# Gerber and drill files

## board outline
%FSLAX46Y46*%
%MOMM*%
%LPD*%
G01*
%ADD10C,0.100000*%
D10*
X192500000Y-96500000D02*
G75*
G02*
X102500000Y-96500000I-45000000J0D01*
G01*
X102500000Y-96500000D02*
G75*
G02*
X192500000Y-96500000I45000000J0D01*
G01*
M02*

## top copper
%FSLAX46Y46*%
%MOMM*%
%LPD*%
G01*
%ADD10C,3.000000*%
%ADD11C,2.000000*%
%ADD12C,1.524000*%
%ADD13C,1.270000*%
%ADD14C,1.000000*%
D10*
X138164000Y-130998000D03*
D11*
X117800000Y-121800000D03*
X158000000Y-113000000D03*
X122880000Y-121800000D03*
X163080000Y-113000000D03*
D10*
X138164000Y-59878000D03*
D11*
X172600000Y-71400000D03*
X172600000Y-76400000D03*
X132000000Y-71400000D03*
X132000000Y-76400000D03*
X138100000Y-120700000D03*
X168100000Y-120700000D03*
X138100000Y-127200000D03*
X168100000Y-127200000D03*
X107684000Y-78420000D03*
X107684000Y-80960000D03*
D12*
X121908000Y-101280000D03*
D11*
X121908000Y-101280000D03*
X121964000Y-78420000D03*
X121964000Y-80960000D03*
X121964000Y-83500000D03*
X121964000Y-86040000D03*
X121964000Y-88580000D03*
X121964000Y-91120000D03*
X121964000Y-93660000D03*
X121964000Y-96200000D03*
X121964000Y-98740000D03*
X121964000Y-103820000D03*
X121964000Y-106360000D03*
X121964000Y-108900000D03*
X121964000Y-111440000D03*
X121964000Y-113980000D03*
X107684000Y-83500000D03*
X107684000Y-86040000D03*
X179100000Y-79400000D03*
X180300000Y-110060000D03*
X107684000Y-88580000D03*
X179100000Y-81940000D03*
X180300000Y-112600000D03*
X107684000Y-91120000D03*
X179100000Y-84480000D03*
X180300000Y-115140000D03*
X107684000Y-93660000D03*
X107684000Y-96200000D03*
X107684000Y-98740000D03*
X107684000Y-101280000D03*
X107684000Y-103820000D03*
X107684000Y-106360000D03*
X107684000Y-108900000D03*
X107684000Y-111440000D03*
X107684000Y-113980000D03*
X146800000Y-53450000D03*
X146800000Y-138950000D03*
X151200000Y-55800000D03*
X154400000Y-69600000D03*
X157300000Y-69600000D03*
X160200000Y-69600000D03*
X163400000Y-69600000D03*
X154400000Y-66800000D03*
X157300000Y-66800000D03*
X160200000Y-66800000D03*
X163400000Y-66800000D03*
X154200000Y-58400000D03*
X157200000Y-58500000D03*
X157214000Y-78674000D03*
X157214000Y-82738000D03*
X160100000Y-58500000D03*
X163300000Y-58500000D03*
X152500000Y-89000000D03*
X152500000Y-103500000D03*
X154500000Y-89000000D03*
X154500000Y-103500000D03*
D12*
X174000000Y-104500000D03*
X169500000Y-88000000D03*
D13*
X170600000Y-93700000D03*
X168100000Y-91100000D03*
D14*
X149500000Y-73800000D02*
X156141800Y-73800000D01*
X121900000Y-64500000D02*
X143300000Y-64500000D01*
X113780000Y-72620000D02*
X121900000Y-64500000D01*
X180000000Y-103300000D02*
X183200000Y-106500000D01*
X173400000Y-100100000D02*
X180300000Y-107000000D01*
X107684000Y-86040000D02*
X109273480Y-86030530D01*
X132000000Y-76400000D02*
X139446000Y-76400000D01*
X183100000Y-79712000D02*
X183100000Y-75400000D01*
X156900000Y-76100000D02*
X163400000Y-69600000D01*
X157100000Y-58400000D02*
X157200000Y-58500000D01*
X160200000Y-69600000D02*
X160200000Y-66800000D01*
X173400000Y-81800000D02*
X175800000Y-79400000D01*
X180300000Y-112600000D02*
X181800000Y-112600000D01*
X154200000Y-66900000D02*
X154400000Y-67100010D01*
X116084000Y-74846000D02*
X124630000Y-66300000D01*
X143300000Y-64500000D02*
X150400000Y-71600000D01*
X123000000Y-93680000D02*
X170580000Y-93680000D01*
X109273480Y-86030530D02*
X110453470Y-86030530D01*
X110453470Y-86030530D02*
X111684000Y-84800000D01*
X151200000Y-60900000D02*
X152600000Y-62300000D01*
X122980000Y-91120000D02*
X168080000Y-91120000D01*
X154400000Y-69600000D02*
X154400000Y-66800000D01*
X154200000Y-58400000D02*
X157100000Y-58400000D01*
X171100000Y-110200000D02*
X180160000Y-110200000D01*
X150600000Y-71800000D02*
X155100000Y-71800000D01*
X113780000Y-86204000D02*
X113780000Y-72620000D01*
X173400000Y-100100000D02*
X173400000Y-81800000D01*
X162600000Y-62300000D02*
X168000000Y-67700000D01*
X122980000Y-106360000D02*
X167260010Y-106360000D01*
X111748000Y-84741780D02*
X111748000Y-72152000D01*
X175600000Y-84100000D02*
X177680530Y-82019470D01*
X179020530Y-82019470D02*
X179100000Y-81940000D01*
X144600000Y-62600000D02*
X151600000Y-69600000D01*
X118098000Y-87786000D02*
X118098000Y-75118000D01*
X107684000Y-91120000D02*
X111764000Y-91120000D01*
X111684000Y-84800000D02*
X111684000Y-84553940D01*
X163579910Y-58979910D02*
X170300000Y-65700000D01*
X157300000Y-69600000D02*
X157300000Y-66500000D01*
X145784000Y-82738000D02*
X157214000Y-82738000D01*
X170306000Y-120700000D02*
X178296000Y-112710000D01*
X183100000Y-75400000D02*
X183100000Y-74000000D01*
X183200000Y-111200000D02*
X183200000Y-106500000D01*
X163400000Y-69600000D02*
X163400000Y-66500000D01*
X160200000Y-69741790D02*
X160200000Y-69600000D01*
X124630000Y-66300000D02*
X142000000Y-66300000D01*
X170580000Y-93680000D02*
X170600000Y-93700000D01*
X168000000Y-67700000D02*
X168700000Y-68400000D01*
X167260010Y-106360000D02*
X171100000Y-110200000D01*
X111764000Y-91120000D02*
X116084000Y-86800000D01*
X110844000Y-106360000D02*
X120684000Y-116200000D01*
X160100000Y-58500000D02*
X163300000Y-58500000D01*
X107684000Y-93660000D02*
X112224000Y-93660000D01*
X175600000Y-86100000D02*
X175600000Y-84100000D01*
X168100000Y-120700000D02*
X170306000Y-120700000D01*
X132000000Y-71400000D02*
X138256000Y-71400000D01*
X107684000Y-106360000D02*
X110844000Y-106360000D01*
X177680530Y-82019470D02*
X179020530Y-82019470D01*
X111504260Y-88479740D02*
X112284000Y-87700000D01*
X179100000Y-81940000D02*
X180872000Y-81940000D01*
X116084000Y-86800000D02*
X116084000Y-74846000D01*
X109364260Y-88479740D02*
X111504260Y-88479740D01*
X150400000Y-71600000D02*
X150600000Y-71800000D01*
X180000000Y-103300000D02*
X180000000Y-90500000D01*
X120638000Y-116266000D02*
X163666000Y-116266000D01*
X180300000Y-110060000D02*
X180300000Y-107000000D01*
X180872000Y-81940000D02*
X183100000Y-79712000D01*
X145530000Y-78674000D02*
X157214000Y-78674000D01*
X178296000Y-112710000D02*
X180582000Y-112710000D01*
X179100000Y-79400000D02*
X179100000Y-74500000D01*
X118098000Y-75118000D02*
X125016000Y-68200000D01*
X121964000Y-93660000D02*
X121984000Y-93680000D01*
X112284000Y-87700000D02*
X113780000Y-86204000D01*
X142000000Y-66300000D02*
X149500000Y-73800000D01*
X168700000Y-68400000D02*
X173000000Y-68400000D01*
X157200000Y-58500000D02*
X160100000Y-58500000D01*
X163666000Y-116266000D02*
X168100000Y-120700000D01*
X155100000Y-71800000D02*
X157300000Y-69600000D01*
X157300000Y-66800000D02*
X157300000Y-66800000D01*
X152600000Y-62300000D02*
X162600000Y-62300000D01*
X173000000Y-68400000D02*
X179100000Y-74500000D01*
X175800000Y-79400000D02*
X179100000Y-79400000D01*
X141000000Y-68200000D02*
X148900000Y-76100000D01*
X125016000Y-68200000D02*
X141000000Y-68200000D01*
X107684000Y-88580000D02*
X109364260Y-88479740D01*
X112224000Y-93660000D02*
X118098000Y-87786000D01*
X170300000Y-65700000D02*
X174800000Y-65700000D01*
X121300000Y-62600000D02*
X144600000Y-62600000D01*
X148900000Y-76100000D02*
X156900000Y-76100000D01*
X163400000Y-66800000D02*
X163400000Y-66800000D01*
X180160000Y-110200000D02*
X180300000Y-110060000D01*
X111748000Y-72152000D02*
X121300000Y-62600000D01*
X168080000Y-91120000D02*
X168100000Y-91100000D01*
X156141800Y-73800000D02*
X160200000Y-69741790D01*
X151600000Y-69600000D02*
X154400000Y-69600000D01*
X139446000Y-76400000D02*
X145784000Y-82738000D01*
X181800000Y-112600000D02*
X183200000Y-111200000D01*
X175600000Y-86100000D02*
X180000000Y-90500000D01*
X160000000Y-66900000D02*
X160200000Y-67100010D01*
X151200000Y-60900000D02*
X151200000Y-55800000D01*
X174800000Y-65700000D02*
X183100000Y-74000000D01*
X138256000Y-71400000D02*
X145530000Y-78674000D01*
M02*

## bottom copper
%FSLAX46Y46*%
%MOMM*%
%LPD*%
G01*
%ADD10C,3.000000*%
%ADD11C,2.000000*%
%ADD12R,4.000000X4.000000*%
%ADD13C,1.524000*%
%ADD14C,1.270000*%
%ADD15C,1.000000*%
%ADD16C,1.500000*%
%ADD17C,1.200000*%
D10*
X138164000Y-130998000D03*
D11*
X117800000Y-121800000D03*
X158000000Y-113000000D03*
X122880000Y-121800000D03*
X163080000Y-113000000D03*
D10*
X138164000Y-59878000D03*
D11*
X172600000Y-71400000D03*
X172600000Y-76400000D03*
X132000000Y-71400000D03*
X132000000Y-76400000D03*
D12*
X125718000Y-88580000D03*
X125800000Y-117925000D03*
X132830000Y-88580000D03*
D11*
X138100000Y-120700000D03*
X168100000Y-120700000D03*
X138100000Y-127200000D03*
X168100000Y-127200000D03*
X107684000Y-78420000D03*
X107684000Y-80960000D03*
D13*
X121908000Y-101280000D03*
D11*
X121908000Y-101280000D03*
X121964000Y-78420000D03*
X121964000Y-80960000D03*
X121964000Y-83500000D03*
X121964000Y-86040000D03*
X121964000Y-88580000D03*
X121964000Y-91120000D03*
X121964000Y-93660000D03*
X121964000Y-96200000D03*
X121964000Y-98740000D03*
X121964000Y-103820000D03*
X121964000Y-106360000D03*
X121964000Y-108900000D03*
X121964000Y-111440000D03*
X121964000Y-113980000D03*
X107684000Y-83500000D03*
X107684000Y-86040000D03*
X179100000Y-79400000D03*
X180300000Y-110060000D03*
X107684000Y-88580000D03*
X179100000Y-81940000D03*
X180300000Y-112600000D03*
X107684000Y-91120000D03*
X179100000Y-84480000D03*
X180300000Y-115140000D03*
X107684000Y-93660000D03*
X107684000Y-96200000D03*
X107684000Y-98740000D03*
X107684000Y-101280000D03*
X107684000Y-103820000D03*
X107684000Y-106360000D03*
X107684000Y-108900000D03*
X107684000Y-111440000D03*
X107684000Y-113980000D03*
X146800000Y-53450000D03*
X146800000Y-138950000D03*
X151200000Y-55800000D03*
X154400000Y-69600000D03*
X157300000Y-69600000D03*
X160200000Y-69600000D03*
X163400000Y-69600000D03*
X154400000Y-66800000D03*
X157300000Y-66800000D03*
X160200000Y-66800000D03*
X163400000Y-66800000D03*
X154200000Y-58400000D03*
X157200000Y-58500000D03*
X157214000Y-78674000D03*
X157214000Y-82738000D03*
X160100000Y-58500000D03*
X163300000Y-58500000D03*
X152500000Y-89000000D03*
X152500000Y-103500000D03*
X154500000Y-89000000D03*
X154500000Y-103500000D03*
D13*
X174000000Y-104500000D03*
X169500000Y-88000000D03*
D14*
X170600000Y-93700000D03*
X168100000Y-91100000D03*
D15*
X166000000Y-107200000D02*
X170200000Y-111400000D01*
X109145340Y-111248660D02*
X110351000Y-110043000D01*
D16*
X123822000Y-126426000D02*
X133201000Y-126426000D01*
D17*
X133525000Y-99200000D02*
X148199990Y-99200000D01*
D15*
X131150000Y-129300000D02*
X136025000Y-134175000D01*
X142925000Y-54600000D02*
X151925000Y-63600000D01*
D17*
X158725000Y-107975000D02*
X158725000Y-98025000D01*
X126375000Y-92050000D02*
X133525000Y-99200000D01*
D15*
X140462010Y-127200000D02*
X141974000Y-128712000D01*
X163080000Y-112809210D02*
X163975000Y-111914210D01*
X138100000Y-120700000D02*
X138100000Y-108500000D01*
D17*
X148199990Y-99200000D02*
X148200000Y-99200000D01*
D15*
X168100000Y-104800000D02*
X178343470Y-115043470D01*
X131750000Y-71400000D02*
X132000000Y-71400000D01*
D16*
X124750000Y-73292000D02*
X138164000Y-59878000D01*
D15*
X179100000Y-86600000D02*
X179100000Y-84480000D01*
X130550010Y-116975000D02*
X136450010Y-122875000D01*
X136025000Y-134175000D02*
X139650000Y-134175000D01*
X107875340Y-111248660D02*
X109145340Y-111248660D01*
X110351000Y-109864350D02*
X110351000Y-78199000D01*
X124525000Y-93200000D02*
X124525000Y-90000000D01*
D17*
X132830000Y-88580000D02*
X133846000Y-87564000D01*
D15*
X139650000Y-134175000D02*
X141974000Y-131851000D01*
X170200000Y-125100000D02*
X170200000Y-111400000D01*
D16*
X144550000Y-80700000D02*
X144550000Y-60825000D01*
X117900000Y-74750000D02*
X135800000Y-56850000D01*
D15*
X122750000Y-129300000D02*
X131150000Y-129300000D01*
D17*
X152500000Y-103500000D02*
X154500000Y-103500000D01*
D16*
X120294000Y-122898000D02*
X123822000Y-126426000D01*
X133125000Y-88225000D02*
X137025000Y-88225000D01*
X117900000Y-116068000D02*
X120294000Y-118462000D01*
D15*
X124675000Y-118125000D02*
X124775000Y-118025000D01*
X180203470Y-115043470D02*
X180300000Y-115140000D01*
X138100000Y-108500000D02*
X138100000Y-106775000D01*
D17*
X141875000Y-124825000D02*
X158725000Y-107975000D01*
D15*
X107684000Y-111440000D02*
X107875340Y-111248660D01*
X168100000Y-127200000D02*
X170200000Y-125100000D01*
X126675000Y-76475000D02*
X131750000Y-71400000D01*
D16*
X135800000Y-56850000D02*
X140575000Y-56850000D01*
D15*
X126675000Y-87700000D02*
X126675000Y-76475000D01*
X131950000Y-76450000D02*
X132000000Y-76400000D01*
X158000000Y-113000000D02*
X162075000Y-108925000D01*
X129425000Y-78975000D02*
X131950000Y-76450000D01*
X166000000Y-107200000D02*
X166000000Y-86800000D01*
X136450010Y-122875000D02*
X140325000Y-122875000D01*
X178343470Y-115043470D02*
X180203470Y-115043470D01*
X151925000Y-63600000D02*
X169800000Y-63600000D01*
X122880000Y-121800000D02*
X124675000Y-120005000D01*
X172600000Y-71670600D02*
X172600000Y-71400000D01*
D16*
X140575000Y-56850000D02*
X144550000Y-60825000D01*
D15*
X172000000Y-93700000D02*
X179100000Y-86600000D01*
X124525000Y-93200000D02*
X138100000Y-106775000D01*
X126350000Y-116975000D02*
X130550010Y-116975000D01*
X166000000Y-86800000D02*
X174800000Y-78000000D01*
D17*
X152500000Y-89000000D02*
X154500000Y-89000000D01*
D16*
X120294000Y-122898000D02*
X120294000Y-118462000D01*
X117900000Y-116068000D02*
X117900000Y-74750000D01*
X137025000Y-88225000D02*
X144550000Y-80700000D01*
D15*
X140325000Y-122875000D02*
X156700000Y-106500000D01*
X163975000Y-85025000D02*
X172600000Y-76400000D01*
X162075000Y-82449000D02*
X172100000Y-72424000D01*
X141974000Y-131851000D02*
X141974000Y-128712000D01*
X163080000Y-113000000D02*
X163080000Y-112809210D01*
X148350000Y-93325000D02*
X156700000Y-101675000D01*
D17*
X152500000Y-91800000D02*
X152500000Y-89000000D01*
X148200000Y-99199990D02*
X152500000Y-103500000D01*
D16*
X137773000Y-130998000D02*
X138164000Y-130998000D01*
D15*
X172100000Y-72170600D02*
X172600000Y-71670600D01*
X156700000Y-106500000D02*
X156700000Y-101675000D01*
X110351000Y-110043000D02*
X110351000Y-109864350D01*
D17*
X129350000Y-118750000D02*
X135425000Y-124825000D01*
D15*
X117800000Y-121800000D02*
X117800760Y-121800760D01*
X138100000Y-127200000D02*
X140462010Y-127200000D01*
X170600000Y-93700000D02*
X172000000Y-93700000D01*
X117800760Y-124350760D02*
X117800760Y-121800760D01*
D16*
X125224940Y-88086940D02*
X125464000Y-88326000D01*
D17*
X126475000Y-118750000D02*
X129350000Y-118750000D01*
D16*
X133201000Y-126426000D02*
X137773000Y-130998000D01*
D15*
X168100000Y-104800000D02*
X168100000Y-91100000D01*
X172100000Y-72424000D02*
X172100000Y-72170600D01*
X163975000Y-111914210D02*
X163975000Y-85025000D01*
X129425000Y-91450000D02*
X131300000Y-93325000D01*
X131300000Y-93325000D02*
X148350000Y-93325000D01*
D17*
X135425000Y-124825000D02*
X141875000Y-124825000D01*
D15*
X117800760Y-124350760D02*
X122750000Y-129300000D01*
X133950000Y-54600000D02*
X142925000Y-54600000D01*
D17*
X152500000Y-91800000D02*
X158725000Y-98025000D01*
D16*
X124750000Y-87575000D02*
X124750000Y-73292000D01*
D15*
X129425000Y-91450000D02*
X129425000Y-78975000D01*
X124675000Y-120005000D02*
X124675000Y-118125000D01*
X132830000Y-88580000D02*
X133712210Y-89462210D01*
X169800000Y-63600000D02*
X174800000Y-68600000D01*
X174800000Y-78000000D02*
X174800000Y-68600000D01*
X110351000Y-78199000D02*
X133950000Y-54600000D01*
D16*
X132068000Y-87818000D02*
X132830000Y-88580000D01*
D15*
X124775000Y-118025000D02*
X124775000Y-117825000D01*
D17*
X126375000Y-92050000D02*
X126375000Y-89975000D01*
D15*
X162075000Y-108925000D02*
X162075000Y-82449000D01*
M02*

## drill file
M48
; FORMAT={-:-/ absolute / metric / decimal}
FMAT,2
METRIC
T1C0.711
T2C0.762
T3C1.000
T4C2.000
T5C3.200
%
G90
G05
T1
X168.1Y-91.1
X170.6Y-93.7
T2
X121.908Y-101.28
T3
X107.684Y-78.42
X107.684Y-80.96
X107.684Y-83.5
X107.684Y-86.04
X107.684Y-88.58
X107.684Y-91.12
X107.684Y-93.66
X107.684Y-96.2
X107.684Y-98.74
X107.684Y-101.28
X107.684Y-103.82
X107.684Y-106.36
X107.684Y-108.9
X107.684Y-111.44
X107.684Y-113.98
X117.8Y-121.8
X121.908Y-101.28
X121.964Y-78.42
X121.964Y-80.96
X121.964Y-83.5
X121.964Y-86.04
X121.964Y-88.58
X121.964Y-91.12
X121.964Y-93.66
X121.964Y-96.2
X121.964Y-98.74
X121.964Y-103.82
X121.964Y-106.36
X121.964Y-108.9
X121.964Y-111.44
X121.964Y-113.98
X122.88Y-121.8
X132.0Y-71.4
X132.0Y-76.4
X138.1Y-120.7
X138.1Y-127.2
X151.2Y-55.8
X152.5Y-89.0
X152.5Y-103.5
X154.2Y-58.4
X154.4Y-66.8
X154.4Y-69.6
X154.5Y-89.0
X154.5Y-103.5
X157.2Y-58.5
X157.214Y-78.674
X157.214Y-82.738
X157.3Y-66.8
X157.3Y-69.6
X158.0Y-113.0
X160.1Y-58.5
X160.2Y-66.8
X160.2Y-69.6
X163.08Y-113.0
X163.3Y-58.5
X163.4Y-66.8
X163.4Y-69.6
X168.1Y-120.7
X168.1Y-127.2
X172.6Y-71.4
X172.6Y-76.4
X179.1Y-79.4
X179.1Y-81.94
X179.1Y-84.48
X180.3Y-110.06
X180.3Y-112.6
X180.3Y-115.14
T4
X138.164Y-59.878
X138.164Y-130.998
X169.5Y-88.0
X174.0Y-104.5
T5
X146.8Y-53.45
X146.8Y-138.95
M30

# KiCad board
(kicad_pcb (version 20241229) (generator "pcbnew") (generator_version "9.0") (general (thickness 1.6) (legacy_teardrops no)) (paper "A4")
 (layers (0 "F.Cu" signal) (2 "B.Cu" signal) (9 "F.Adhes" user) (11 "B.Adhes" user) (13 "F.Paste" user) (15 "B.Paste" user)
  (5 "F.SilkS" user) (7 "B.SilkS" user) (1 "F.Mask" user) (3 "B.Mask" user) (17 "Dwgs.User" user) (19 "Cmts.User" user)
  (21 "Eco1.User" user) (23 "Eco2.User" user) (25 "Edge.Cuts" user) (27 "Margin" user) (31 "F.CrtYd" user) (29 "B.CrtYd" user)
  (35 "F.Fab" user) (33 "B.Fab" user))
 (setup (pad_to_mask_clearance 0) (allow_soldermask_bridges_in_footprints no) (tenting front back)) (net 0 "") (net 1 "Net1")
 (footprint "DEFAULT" (layer "F.Cu") (at 51.8 171.2)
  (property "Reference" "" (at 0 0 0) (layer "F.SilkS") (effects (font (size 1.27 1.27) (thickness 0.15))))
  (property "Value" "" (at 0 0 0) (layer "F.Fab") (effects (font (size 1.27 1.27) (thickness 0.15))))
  (pad "" thru_hole circle (at 86.364 -40.202) (size 3 3) (drill 2) (layers "*.Cu") (remove_unused_layers no))
  (pad "105" thru_hole circle (at 66 -49.4) (size 2 2) (drill 1) (layers "*.Cu") (remove_unused_layers no))
  (pad "105" thru_hole circle (at 106.2 -58.2) (size 2 2) (drill 1) (layers "*.Cu") (remove_unused_layers no))
  (pad "107" thru_hole circle (at 71.08 -49.4) (size 2 2) (drill 1) (layers "*.Cu") (remove_unused_layers no))
  (pad "107" thru_hole circle (at 111.28 -58.2) (size 2 2) (drill 1) (layers "*.Cu") (remove_unused_layers no))
  (pad "128" thru_hole circle (at 86.364 -111.322) (size 3 3) (drill 2) (layers "*.Cu") (remove_unused_layers no))
  (pad "129" thru_hole circle (at 120.8 -99.8 270) (size 2 2) (drill 1) (layers "*.Cu") (remove_unused_layers no))
  (pad "130" thru_hole circle (at 120.8 -94.8 270) (size 2 2) (drill 1) (layers "*.Cu") (remove_unused_layers no))
  (pad "131" thru_hole circle (at 80.2 -99.8 270) (size 2 2) (drill 1) (layers "*.Cu") (remove_unused_layers no))
  (pad "132" thru_hole circle (at 80.2 -94.8 270) (size 2 2) (drill 1) (layers "*.Cu") (remove_unused_layers no))
  (pad "134" smd rect (at 73.918 -82.62) (size 4 4) (layers "B.Cu"))
  (pad "134" smd rect (at 74 -53.275) (size 4 4) (layers "B.Cu"))
  (pad "134" smd rect (at 81.03 -82.62) (size 4 4) (layers "B.Cu"))
  (pad "137" thru_hole circle (at 86.3 -50.5 270) (size 2 2) (drill 1) (layers "*.Cu") (remove_unused_layers no))
  (pad "137" thru_hole circle (at 116.3 -50.5 270) (size 2 2) (drill 1) (layers "*.Cu") (remove_unused_layers no))
  (pad "138" thru_hole circle (at 86.3 -44 270) (size 2 2) (drill 1) (layers "*.Cu") (remove_unused_layers no))
  (pad "138" thru_hole circle (at 116.3 -44 270) (size 2 2) (drill 1) (layers "*.Cu") (remove_unused_layers no))
  (pad "141" thru_hole circle (at 55.884 -92.78) (size 2 2) (drill 1) (layers "*.Cu") (remove_unused_layers no))
  (pad "141" thru_hole circle (at 55.884 -90.24) (size 2 2) (drill 1) (layers "*.Cu") (remove_unused_layers no))
  (pad "141" thru_hole circle (at 70.108 -69.92) (size 1.524 1.524) (drill 0.762) (layers "*.Cu") (remove_unused_layers no))
  (pad "141" thru_hole circle (at 70.108 -69.92) (size 2 2) (drill 1) (layers "*.Cu") (remove_unused_layers no))
  (pad "141" thru_hole circle (at 70.164 -92.78) (size 2 2) (drill 1) (layers "*.Cu") (remove_unused_layers no))
  (pad "141" thru_hole circle (at 70.164 -90.24) (size 2 2) (drill 1) (layers "*.Cu") (remove_unused_layers no))
  (pad "141" thru_hole circle (at 70.164 -87.7) (size 2 2) (drill 1) (layers "*.Cu") (remove_unused_layers no))
  (pad "141" thru_hole circle (at 70.164 -85.16) (size 2 2) (drill 1) (layers "*.Cu") (remove_unused_layers no))
  (pad "141" thru_hole circle (at 70.164 -82.62) (size 2 2) (drill 1) (layers "*.Cu") (remove_unused_layers no))
  (pad "141" thru_hole circle (at 70.164 -80.08) (size 2 2) (drill 1) (layers "*.Cu") (remove_unused_layers no))
  (pad "141" thru_hole circle (at 70.164 -77.54) (size 2 2) (drill 1) (layers "*.Cu") (remove_unused_layers no))
  (pad "141" thru_hole circle (at 70.164 -75) (size 2 2) (drill 1) (layers "*.Cu") (remove_unused_layers no))
  (pad "141" thru_hole circle (at 70.164 -72.46) (size 2 2) (drill 1) (layers "*.Cu") (remove_unused_layers no))
  (pad "141" thru_hole circle (at 70.164 -67.38) (size 2 2) (drill 1) (layers "*.Cu") (remove_unused_layers no))
  (pad "141" thru_hole circle (at 70.164 -64.84) (size 2 2) (drill 1) (layers "*.Cu") (remove_unused_layers no))
  (pad "141" thru_hole circle (at 70.164 -62.3) (size 2 2) (drill 1) (layers "*.Cu") (remove_unused_layers no))
  (pad "141" thru_hole circle (at 70.164 -59.76) (size 2 2) (drill 1) (layers "*.Cu") (remove_unused_layers no))
  (pad "141" thru_hole circle (at 70.164 -57.22) (size 2 2) (drill 1) (layers "*.Cu") (remove_unused_layers no))
  (pad "142" thru_hole circle (at 55.884 -87.7) (size 2 2) (drill 1) (layers "*.Cu") (remove_unused_layers no))
  (pad "143" thru_hole circle (at 55.884 -85.16) (size 2 2) (drill 1) (layers "*.Cu") (remove_unused_layers no))
  (pad "143" thru_hole circle (at 127.3 -91.8) (size 2 2) (drill 1) (layers "*.Cu") (remove_unused_layers no))
  (pad "143" thru_hole circle (at 128.5 -61.14) (size 2 2) (drill 1) (layers "*.Cu") (remove_unused_layers no))
  (pad "144" thru_hole circle (at 55.884 -82.62) (size 2 2) (drill 1) (layers "*.Cu") (remove_unused_layers no))
  (pad "144" thru_hole circle (at 127.3 -89.26) (size 2 2) (drill 1) (layers "*.Cu") (remove_unused_layers no))
  (pad "144" thru_hole circle (at 128.5 -58.6) (size 2 2) (drill 1) (layers "*.Cu") (remove_unused_layers no))
  (pad "145" thru_hole circle (at 55.884 -80.08) (size 2 2) (drill 1) (layers "*.Cu") (remove_unused_layers no))
  (pad "145" thru_hole circle (at 127.3 -86.72) (size 2 2) (drill 1) (layers "*.Cu") (remove_unused_layers no))
  (pad "145" thru_hole circle (at 128.5 -56.06) (size 2 2) (drill 1) (layers "*.Cu") (remove_unused_layers no))
  (pad "146" thru_hole circle (at 55.884 -77.54) (size 2 2) (drill 1) (layers "*.Cu") (remove_unused_layers no))
  (pad "147" thru_hole circle (at 55.884 -75) (size 2 2) (drill 1) (layers "*.Cu") (remove_unused_layers no))
  (pad "148" thru_hole circle (at 55.884 -72.46) (size 2 2) (drill 1) (layers "*.Cu") (remove_unused_layers no))
  (pad "149" thru_hole circle (at 55.884 -69.92) (size 2 2) (drill 1) (layers "*.Cu") (remove_unused_layers no))
  (pad "150" thru_hole circle (at 55.884 -67.38) (size 2 2) (drill 1) (layers "*.Cu") (remove_unused_layers no))
  (pad "151" thru_hole circle (at 55.884 -64.84) (size 2 2) (drill 1) (layers "*.Cu") (remove_unused_layers no))
  (pad "152" thru_hole circle (at 55.884 -62.3) (size 2 2) (drill 1) (layers "*.Cu") (remove_unused_layers no))
  (pad "153" thru_hole circle (at 55.884 -59.76) (size 2 2) (drill 1) (layers "*.Cu") (remove_unused_layers no))
  (pad "154" thru_hole circle (at 55.884 -57.22) (size 2 2) (drill 1) (layers "*.Cu") (remove_unused_layers no))
  (pad "155" thru_hole circle (at 95 -117.75) (size 2 2) (drill 3.2) (layers "*.Cu") (remove_unused_layers no))
  (pad "155" thru_hole circle (at 95 -32.25) (size 2 2) (drill 3.2) (layers "*.Cu") (remove_unused_layers no))
  (pad "155" thru_hole circle (at 99.4 -115.4) (size 2 2) (drill 1) (layers "*.Cu") (remove_unused_layers no))
  (pad "156" thru_hole circle (at 102.6 -101.6) (size 2 2) (drill 1) (layers "*.Cu") (remove_unused_layers no))
  (pad "156" thru_hole circle (at 105.5 -101.6) (size 2 2) (drill 1) (layers "*.Cu") (remove_unused_layers no))
  (pad "156" thru_hole circle (at 108.4 -101.6) (size 2 2) (drill 1) (layers "*.Cu") (remove_unused_layers no))
  (pad "156" thru_hole circle (at 111.6 -101.6) (size 2 2) (drill 1) (layers "*.Cu") (remove_unused_layers no))
  (pad "157" thru_hole circle (at 102.6 -104.4) (size 2 2) (drill 1) (layers "*.Cu") (remove_unused_layers no))
  (pad "157" thru_hole circle (at 105.5 -104.4) (size 2 2) (drill 1) (layers "*.Cu") (remove_unused_layers no))
  (pad "157" thru_hole circle (at 108.4 -104.4) (size 2 2) (drill 1) (layers "*.Cu") (remove_unused_layers no))
  (pad "157" thru_hole circle (at 111.6 -104.4) (size 2 2) (drill 1) (layers "*.Cu") (remove_unused_layers no))
  (pad "158" thru_hole circle (at 102.4 -112.8) (size 2 2) (drill 1) (layers "*.Cu") (remove_unused_layers no))
  (pad "158" thru_hole circle (at 105.4 -112.7) (size 2 2) (drill 1) (layers "*.Cu") (remove_unused_layers no))
  (pad "158" thru_hole circle (at 105.414 -92.526) (size 2 2) (drill 1) (layers "*.Cu") (remove_unused_layers no))
  (pad "158" thru_hole circle (at 105.414 -88.462) (size 2 2) (drill 1) (layers "*.Cu") (remove_unused_layers no))
  (pad "158" thru_hole circle (at 108.3 -112.7) (size 2 2) (drill 1) (layers "*.Cu") (remove_unused_layers no))
  (pad "158" thru_hole circle (at 111.5 -112.7) (size 2 2) (drill 1) (layers "*.Cu") (remove_unused_layers no))
  (pad "169" thru_hole circle (at 100.7 -82.2) (size 2 2) (drill 1) (layers "*.Cu") (remove_unused_layers no))
  (pad "169" thru_hole circle (at 100.7 -67.7) (size 2 2) (drill 1) (layers "*.Cu") (remove_unused_layers no))
  (pad "170" thru_hole circle (at 102.7 -82.2) (size 2 2) (drill 1) (layers "*.Cu") (remove_unused_layers no))
  (pad "170" thru_hole circle (at 102.7 -67.7) (size 2 2) (drill 1) (layers "*.Cu") (remove_unused_layers no))
  (pad "171" thru_hole circle (at 122.2 -66.7) (size 1.524 1.524) (drill 2) (layers "*.Cu") (remove_unused_layers no))
  (pad "172" thru_hole circle (at 117.7 -83.2) (size 1.524 1.524) (drill 2) (layers "*.Cu") (remove_unused_layers no)))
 (gr_circle (center 147.5 96.5) (end 192.5 96.5) (stroke (width 0.1) (type solid)) (fill no) (layer "Edge.Cuts"))
 (segment (start 149.5 73.8) (end 156.1418 73.8) (width 1) (layer "F.Cu") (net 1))
 (segment (start 121.9 64.5) (end 143.3 64.5) (width 1) (layer "F.Cu") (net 1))
 (segment (start 113.78 72.62) (end 121.9 64.5) (width 1) (layer "F.Cu") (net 1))
 (segment (start 180 103.3) (end 183.2 106.5) (width 1) (layer "F.Cu") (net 1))
 (segment (start 173.4 100.1) (end 180.3 107) (width 1) (layer "F.Cu") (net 1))
 (segment (start 107.684 86.04) (end 109.27348 86.03053) (width 1) (layer "F.Cu") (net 1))
 (segment (start 132 76.4) (end 139.446 76.4) (width 1) (layer "F.Cu") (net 1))
 (segment (start 183.1 79.712) (end 183.1 75.4) (width 1) (layer "F.Cu") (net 1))
 (segment (start 156.9 76.1) (end 163.4 69.6) (width 1) (layer "F.Cu") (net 1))
 (segment (start 157.1 58.4) (end 157.2 58.5) (width 1) (layer "F.Cu") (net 1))
 (segment (start 160.2 69.6) (end 160.2 66.8) (width 1) (layer "F.Cu") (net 1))
 (segment (start 173.4 81.8) (end 175.8 79.4) (width 1) (layer "F.Cu") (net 1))
 (segment (start 180.3 112.6) (end 181.8 112.6) (width 1) (layer "F.Cu") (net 1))
 (segment (start 154.2 66.9) (end 154.4 67.10001) (width 1) (layer "F.Cu") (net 1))
 (segment (start 116.084 74.846) (end 124.63 66.3) (width 1) (layer "F.Cu") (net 1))
 (segment (start 143.3 64.5) (end 150.4 71.6) (width 1) (layer "F.Cu") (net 1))
 (segment (start 123 93.68) (end 170.58 93.68) (width 1) (layer "F.Cu") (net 1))
 (segment (start 109.27348 86.03053) (end 110.45347 86.03053) (width 1) (layer "F.Cu") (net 1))
 (segment (start 110.45347 86.03053) (end 111.684 84.8) (width 1) (layer "F.Cu") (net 1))
 (segment (start 151.2 60.9) (end 152.6 62.3) (width 1) (layer "F.Cu") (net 1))
 (segment (start 122.98 91.12) (end 168.08 91.12) (width 1) (layer "F.Cu") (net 1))
 (segment (start 154.4 69.6) (end 154.4 66.8) (width 1) (layer "F.Cu") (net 1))
 (segment (start 154.2 58.4) (end 157.1 58.4) (width 1) (layer "F.Cu") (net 1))
 (segment (start 171.1 110.2) (end 180.16 110.2) (width 1) (layer "F.Cu") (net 1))
 (segment (start 150.6 71.8) (end 155.1 71.8) (width 1) (layer "F.Cu") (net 1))
 (segment (start 113.78 86.204) (end 113.78 72.62) (width 1) (layer "F.Cu") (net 1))
 (segment (start 173.4 100.1) (end 173.4 81.8) (width 1) (layer "F.Cu") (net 1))
 (segment (start 162.6 62.3) (end 168 67.7) (width 1) (layer "F.Cu") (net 1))
 (segment (start 122.98 106.36) (end 167.26001 106.36) (width 1) (layer "F.Cu") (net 1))
 (segment (start 111.748 84.74178) (end 111.748 72.152) (width 1) (layer "F.Cu") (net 1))
 (segment (start 175.6 84.1) (end 177.68053 82.01947) (width 1) (layer "F.Cu") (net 1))
 (segment (start 179.02053 82.01947) (end 179.1 81.94) (width 1) (layer "F.Cu") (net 1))
 (segment (start 144.6 62.6) (end 151.6 69.6) (width 1) (layer "F.Cu") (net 1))
 (segment (start 118.098 87.786) (end 118.098 75.118) (width 1) (layer "F.Cu") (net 1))
 (segment (start 107.684 91.12) (end 111.764 91.12) (width 1) (layer "F.Cu") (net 1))
 (segment (start 111.684 84.8) (end 111.684 84.55394) (width 1) (layer "F.Cu") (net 1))
 (segment (start 163.57991 58.97991) (end 170.3 65.7) (width 1) (layer "F.Cu") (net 1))
 (segment (start 157.3 69.6) (end 157.3 66.5) (width 1) (layer "F.Cu") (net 1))
 (segment (start 145.784 82.738) (end 157.214 82.738) (width 1) (layer "F.Cu") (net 1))
 (segment (start 170.306 120.7) (end 178.296 112.71) (width 1) (layer "F.Cu") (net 1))
 (segment (start 183.1 75.4) (end 183.1 74) (width 1) (layer "F.Cu") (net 1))
 (segment (start 183.2 111.2) (end 183.2 106.5) (width 1) (layer "F.Cu") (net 1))
 (segment (start 163.4 69.6) (end 163.4 66.5) (width 1) (layer "F.Cu") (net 1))
 (segment (start 160.2 69.74179) (end 160.2 69.6) (width 1) (layer "F.Cu") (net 1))
 (segment (start 124.63 66.3) (end 142 66.3) (width 1) (layer "F.Cu") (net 1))
 (segment (start 170.58 93.68) (end 170.6 93.7) (width 1) (layer "F.Cu") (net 1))
 (segment (start 168 67.7) (end 168.7 68.4) (width 1) (layer "F.Cu") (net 1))
 (segment (start 167.26001 106.36) (end 171.1 110.2) (width 1) (layer "F.Cu") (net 1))
 (segment (start 111.764 91.12) (end 116.084 86.8) (width 1) (layer "F.Cu") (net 1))
 (segment (start 110.844 106.36) (end 120.684 116.2) (width 1) (layer "F.Cu") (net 1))
 (segment (start 160.1 58.5) (end 163.3 58.5) (width 1) (layer "F.Cu") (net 1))
 (segment (start 107.684 93.66) (end 112.224 93.66) (width 1) (layer "F.Cu") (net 1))
 (segment (start 175.6 86.1) (end 175.6 84.1) (width 1) (layer "F.Cu") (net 1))
 (segment (start 168.1 120.7) (end 170.306 120.7) (width 1) (layer "F.Cu") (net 1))
 (segment (start 132 71.4) (end 138.256 71.4) (width 1) (layer "F.Cu") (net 1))
 (segment (start 107.684 106.36) (end 110.844 106.36) (width 1) (layer "F.Cu") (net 1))
 (segment (start 177.68053 82.01947) (end 179.02053 82.01947) (width 1) (layer "F.Cu") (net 1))
 (segment (start 111.50426 88.47974) (end 112.284 87.7) (width 1) (layer "F.Cu") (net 1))
 (segment (start 179.1 81.94) (end 180.872 81.94) (width 1) (layer "F.Cu") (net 1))
 (segment (start 116.084 86.8) (end 116.084 74.846) (width 1) (layer "F.Cu") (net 1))
 (segment (start 109.36426 88.47974) (end 111.50426 88.47974) (width 1) (layer "F.Cu") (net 1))
 (segment (start 150.4 71.6) (end 150.6 71.8) (width 1) (layer "F.Cu") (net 1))
 (segment (start 180 103.3) (end 180 90.5) (width 1) (layer "F.Cu") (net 1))
 (segment (start 120.638 116.266) (end 163.666 116.266) (width 1) (layer "F.Cu") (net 1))
 (segment (start 180.3 110.06) (end 180.3 107) (width 1) (layer "F.Cu") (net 1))
 (segment (start 180.872 81.94) (end 183.1 79.712) (width 1) (layer "F.Cu") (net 1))
 (segment (start 145.53 78.674) (end 157.214 78.674) (width 1) (layer "F.Cu") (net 1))
 (segment (start 178.296 112.71) (end 180.582 112.71) (width 1) (layer "F.Cu") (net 1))
 (segment (start 179.1 79.4) (end 179.1 74.5) (width 1) (layer "F.Cu") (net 1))
 (segment (start 118.098 75.118) (end 125.016 68.2) (width 1) (layer "F.Cu") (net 1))
 (segment (start 121.964 93.66) (end 121.984 93.68) (width 1) (layer "F.Cu") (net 1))
 (segment (start 112.284 87.7) (end 113.78 86.204) (width 1) (layer "F.Cu") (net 1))
 (segment (start 142 66.3) (end 149.5 73.8) (width 1) (layer "F.Cu") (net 1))
 (segment (start 168.7 68.4) (end 173 68.4) (width 1) (layer "F.Cu") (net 1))
 (segment (start 157.2 58.5) (end 160.1 58.5) (width 1) (layer "F.Cu") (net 1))
 (segment (start 163.666 116.266) (end 168.1 120.7) (width 1) (layer "F.Cu") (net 1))
 (segment (start 155.1 71.8) (end 157.3 69.6) (width 1) (layer "F.Cu") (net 1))
 (segment (start 157.3 66.8) (end 157.3 66.8) (width 1) (layer "F.Cu") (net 1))
 (segment (start 152.6 62.3) (end 162.6 62.3) (width 1) (layer "F.Cu") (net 1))
 (segment (start 173 68.4) (end 179.1 74.5) (width 1) (layer "F.Cu") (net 1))
 (segment (start 175.8 79.4) (end 179.1 79.4) (width 1) (layer "F.Cu") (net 1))
 (segment (start 141 68.2) (end 148.9 76.1) (width 1) (layer "F.Cu") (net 1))
 (segment (start 125.016 68.2) (end 141 68.2) (width 1) (layer "F.Cu") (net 1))
 (segment (start 107.684 88.58) (end 109.36426 88.47974) (width 1) (layer "F.Cu") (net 1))
 (segment (start 112.224 93.66) (end 118.098 87.786) (width 1) (layer "F.Cu") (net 1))
 (segment (start 170.3 65.7) (end 174.8 65.7) (width 1) (layer "F.Cu") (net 1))
 (segment (start 121.3 62.6) (end 144.6 62.6) (width 1) (layer "F.Cu") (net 1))
 (segment (start 148.9 76.1) (end 156.9 76.1) (width 1) (layer "F.Cu") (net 1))
 (segment (start 163.4 66.8) (end 163.4 66.8) (width 1) (layer "F.Cu") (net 1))
 (segment (start 180.16 110.2) (end 180.3 110.06) (width 1) (layer "F.Cu") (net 1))
 (segment (start 111.748 72.152) (end 121.3 62.6) (width 1) (layer "F.Cu") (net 1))
 (segment (start 168.08 91.12) (end 168.1 91.1) (width 1) (layer "F.Cu") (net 1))
 (segment (start 156.1418 73.8) (end 160.2 69.74179) (width 1) (layer "F.Cu") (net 1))
 (segment (start 151.6 69.6) (end 154.4 69.6) (width 1) (layer "F.Cu") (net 1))
 (segment (start 139.446 76.4) (end 145.784 82.738) (width 1) (layer "F.Cu") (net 1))
 (segment (start 181.8 112.6) (end 183.2 111.2) (width 1) (layer "F.Cu") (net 1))
 (segment (start 175.6 86.1) (end 180 90.5) (width 1) (layer "F.Cu") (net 1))
 (segment (start 160 66.9) (end 160.2 67.10001) (width 1) (layer "F.Cu") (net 1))
 (segment (start 151.2 60.9) (end 151.2 55.8) (width 1) (layer "F.Cu") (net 1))
 (segment (start 174.8 65.7) (end 183.1 74) (width 1) (layer "F.Cu") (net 1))
 (segment (start 138.256 71.4) (end 145.53 78.674) (width 1) (layer "F.Cu") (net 1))
 (via (at 170.6 93.7) (size 1.27) (drill 0.7112) (layers "F.Cu" "B.Cu") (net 1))
 (via (at 168.1 91.1) (size 1.27) (drill 0.7112) (layers "F.Cu" "B.Cu") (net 1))
 (segment (start 166 107.2) (end 170.2 111.4) (width 1) (layer "B.Cu") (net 1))
 (segment (start 109.14534 111.24866) (end 110.351 110.043) (width 1) (layer "B.Cu") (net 1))
 (segment (start 123.822 126.426) (end 133.201 126.426) (width 1.5) (layer "B.Cu") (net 1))
 (segment (start 133.525 99.2) (end 148.19999 99.2) (width 1.2) (layer "B.Cu") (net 1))
 (segment (start 131.15 129.3) (end 136.025 134.175) (width 1) (layer "B.Cu") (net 1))
 (segment (start 142.925 54.6) (end 151.925 63.6) (width 1) (layer "B.Cu") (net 1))
 (segment (start 158.725 107.975) (end 158.725 98.025) (width 1.2) (layer "B.Cu") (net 1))
 (segment (start 126.375 92.05) (end 133.525 99.2) (width 1.2) (layer "B.Cu") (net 1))
 (segment (start 140.46201 127.2) (end 141.974 128.712) (width 1) (layer "B.Cu") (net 1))
 (segment (start 163.08 112.80921) (end 163.975 111.91421) (width 1) (layer "B.Cu") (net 1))
 (segment (start 138.1 120.7) (end 138.1 108.5) (width 1) (layer "B.Cu") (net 1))
 (segment (start 148.19999 99.2) (end 148.2 99.2) (width 1.2) (layer "B.Cu") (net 1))
 (segment (start 168.1 104.8) (end 178.34347 115.04347) (width 1) (layer "B.Cu") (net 1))
 (segment (start 131.75 71.4) (end 132 71.4) (width 1) (layer "B.Cu") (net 1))
 (segment (start 124.75 73.292) (end 138.164 59.878) (width 1.5) (layer "B.Cu") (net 1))
 (segment (start 179.1 86.6) (end 179.1 84.48) (width 1) (layer "B.Cu") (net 1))
 (segment (start 130.55001 116.975) (end 136.45001 122.875) (width 1) (layer "B.Cu") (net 1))
 (segment (start 136.025 134.175) (end 139.65 134.175) (width 1) (layer "B.Cu") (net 1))
 (segment (start 107.87534 111.24866) (end 109.14534 111.24866) (width 1) (layer "B.Cu") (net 1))
 (segment (start 110.351 109.86435) (end 110.351 78.199) (width 1) (layer "B.Cu") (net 1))
 (segment (start 124.525 93.2) (end 124.525 90) (width 1) (layer "B.Cu") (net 1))
 (segment (start 132.83 88.58) (end 133.846 87.564) (width 1.2) (layer "B.Cu") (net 1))
 (segment (start 139.65 134.175) (end 141.974 131.851) (width 1) (layer "B.Cu") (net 1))
 (segment (start 170.2 125.1) (end 170.2 111.4) (width 1) (layer "B.Cu") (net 1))
 (segment (start 144.55 80.7) (end 144.55 60.825) (width 1.5) (layer "B.Cu") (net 1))
 (segment (start 117.9 74.75) (end 135.8 56.85) (width 1.5) (layer "B.Cu") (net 1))
 (segment (start 122.75 129.3) (end 131.15 129.3) (width 1) (layer "B.Cu") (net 1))
 (segment (start 152.5 103.5) (end 154.5 103.5) (width 1.2) (layer "B.Cu") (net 1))
 (segment (start 120.294 122.898) (end 123.822 126.426) (width 1.5) (layer "B.Cu") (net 1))
 (segment (start 133.125 88.225) (end 137.025 88.225) (width 1.5) (layer "B.Cu") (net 1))
 (segment (start 117.9 116.068) (end 120.294 118.462) (width 1.5) (layer "B.Cu") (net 1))
 (segment (start 124.675 118.125) (end 124.775 118.025) (width 1) (layer "B.Cu") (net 1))
 (segment (start 180.20347 115.04347) (end 180.3 115.14) (width 1) (layer "B.Cu") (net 1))
 (segment (start 138.1 108.5) (end 138.1 106.775) (width 1) (layer "B.Cu") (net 1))
 (segment (start 141.875 124.825) (end 158.725 107.975) (width 1.2) (layer "B.Cu") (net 1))
 (segment (start 107.684 111.44) (end 107.87534 111.24866) (width 1) (layer "B.Cu") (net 1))
 (segment (start 168.1 127.2) (end 170.2 125.1) (width 1) (layer "B.Cu") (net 1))
 (segment (start 126.675 76.475) (end 131.75 71.4) (width 1) (layer "B.Cu") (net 1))
 (segment (start 135.8 56.85) (end 140.575 56.85) (width 1.5) (layer "B.Cu") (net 1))
 (segment (start 126.675 87.7) (end 126.675 76.475) (width 1) (layer "B.Cu") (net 1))
 (segment (start 131.95 76.45) (end 132 76.4) (width 1) (layer "B.Cu") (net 1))
 (segment (start 158 113) (end 162.075 108.925) (width 1) (layer "B.Cu") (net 1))
 (segment (start 129.425 78.975) (end 131.95 76.45) (width 1) (layer "B.Cu") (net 1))
 (segment (start 166 107.2) (end 166 86.8) (width 1) (layer "B.Cu") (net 1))
 (segment (start 136.45001 122.875) (end 140.325 122.875) (width 1) (layer "B.Cu") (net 1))
 (segment (start 178.34347 115.04347) (end 180.20347 115.04347) (width 1) (layer "B.Cu") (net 1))
 (segment (start 151.925 63.6) (end 169.8 63.6) (width 1) (layer "B.Cu") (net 1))
 (segment (start 122.88 121.8) (end 124.675 120.005) (width 1) (layer "B.Cu") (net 1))
 (segment (start 172.6 71.6706) (end 172.6 71.4) (width 1) (layer "B.Cu") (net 1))
 (segment (start 140.575 56.85) (end 144.55 60.825) (width 1.5) (layer "B.Cu") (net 1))
 (segment (start 172 93.7) (end 179.1 86.6) (width 1) (layer "B.Cu") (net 1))
 (segment (start 124.525 93.2) (end 138.1 106.775) (width 1) (layer "B.Cu") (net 1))
 (segment (start 126.35 116.975) (end 130.55001 116.975) (width 1) (layer "B.Cu") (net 1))
 (segment (start 166 86.8) (end 174.8 78) (width 1) (layer "B.Cu") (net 1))
 (segment (start 152.5 89) (end 154.5 89) (width 1.2) (layer "B.Cu") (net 1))
 (segment (start 120.294 122.898) (end 120.294 118.462) (width 1.5) (layer "B.Cu") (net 1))
 (segment (start 117.9 116.068) (end 117.9 74.75) (width 1.5) (layer "B.Cu") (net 1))
 (segment (start 137.025 88.225) (end 144.55 80.7) (width 1.5) (layer "B.Cu") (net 1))
 (segment (start 140.325 122.875) (end 156.7 106.5) (width 1) (layer "B.Cu") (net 1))
 (segment (start 163.975 85.025) (end 172.6 76.4) (width 1) (layer "B.Cu") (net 1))
 (segment (start 162.075 82.449) (end 172.1 72.424) (width 1) (layer "B.Cu") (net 1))
 (segment (start 141.974 131.851) (end 141.974 128.712) (width 1) (layer "B.Cu") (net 1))
 (segment (start 163.08 113) (end 163.08 112.80921) (width 1) (layer "B.Cu") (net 1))
 (segment (start 148.35 93.325) (end 156.7 101.675) (width 1) (layer "B.Cu") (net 1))
 (segment (start 152.5 91.8) (end 152.5 89) (width 1.2) (layer "B.Cu") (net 1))
 (segment (start 148.2 99.19999) (end 152.5 103.5) (width 1.2) (layer "B.Cu") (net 1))
 (segment (start 137.773 130.998) (end 138.164 130.998) (width 1.5) (layer "B.Cu") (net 1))
 (segment (start 172.1 72.1706) (end 172.6 71.6706) (width 1) (layer "B.Cu") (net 1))
 (segment (start 156.7 106.5) (end 156.7 101.675) (width 1) (layer "B.Cu") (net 1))
 (segment (start 110.351 110.043) (end 110.351 109.86435) (width 1) (layer "B.Cu") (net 1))
 (segment (start 129.35 118.75) (end 135.425 124.825) (width 1.2) (layer "B.Cu") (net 1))
 (segment (start 117.8 121.8) (end 117.80076 121.80076) (width 1) (layer "B.Cu") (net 1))
 (segment (start 138.1 127.2) (end 140.46201 127.2) (width 1) (layer "B.Cu") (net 1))
 (segment (start 170.6 93.7) (end 172 93.7) (width 1) (layer "B.Cu") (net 1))
 (segment (start 117.80076 124.35076) (end 117.80076 121.80076) (width 1) (layer "B.Cu") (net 1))
 (segment (start 125.22494 88.08694) (end 125.464 88.326) (width 1.5) (layer "B.Cu") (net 1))
 (segment (start 126.475 118.75) (end 129.35 118.75) (width 1.2) (layer "B.Cu") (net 1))
 (segment (start 133.201 126.426) (end 137.773 130.998) (width 1.5) (layer "B.Cu") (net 1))
 (segment (start 168.1 104.8) (end 168.1 91.1) (width 1) (layer "B.Cu") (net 1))
 (segment (start 172.1 72.424) (end 172.1 72.1706) (width 1) (layer "B.Cu") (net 1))
 (segment (start 163.975 111.91421) (end 163.975 85.025) (width 1) (layer "B.Cu") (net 1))
 (segment (start 129.425 91.45) (end 131.3 93.325) (width 1) (layer "B.Cu") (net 1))
 (segment (start 131.3 93.325) (end 148.35 93.325) (width 1) (layer "B.Cu") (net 1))
 (segment (start 135.425 124.825) (end 141.875 124.825) (width 1.2) (layer "B.Cu") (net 1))
 (segment (start 117.80076 124.35076) (end 122.75 129.3) (width 1) (layer "B.Cu") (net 1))
 (segment (start 133.95 54.6) (end 142.925 54.6) (width 1) (layer "B.Cu") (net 1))
 (segment (start 152.5 91.8) (end 158.725 98.025) (width 1.2) (layer "B.Cu") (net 1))
 (segment (start 124.75 87.575) (end 124.75 73.292) (width 1.5) (layer "B.Cu") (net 1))
 (segment (start 129.425 91.45) (end 129.425 78.975) (width 1) (layer "B.Cu") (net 1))
 (segment (start 124.675 120.005) (end 124.675 118.125) (width 1) (layer "B.Cu") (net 1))
 (segment (start 132.83 88.58) (end 133.71221 89.46221) (width 1) (layer "B.Cu") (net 1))
 (segment (start 169.8 63.6) (end 174.8 68.6) (width 1) (layer "B.Cu") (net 1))
 (segment (start 174.8 78) (end 174.8 68.6) (width 1) (layer "B.Cu") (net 1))
 (segment (start 110.351 78.199) (end 133.95 54.6) (width 1) (layer "B.Cu") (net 1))
 (segment (start 132.068 87.818) (end 132.83 88.58) (width 1.5) (layer "B.Cu") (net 1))
 (segment (start 124.775 118.025) (end 124.775 117.825) (width 1) (layer "B.Cu") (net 1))
 (segment (start 126.375 92.05) (end 126.375 89.975) (width 1.2) (layer "B.Cu") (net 1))
 (segment (start 162.075 108.925) (end 162.075 82.449) (width 1) (layer "B.Cu") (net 1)))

